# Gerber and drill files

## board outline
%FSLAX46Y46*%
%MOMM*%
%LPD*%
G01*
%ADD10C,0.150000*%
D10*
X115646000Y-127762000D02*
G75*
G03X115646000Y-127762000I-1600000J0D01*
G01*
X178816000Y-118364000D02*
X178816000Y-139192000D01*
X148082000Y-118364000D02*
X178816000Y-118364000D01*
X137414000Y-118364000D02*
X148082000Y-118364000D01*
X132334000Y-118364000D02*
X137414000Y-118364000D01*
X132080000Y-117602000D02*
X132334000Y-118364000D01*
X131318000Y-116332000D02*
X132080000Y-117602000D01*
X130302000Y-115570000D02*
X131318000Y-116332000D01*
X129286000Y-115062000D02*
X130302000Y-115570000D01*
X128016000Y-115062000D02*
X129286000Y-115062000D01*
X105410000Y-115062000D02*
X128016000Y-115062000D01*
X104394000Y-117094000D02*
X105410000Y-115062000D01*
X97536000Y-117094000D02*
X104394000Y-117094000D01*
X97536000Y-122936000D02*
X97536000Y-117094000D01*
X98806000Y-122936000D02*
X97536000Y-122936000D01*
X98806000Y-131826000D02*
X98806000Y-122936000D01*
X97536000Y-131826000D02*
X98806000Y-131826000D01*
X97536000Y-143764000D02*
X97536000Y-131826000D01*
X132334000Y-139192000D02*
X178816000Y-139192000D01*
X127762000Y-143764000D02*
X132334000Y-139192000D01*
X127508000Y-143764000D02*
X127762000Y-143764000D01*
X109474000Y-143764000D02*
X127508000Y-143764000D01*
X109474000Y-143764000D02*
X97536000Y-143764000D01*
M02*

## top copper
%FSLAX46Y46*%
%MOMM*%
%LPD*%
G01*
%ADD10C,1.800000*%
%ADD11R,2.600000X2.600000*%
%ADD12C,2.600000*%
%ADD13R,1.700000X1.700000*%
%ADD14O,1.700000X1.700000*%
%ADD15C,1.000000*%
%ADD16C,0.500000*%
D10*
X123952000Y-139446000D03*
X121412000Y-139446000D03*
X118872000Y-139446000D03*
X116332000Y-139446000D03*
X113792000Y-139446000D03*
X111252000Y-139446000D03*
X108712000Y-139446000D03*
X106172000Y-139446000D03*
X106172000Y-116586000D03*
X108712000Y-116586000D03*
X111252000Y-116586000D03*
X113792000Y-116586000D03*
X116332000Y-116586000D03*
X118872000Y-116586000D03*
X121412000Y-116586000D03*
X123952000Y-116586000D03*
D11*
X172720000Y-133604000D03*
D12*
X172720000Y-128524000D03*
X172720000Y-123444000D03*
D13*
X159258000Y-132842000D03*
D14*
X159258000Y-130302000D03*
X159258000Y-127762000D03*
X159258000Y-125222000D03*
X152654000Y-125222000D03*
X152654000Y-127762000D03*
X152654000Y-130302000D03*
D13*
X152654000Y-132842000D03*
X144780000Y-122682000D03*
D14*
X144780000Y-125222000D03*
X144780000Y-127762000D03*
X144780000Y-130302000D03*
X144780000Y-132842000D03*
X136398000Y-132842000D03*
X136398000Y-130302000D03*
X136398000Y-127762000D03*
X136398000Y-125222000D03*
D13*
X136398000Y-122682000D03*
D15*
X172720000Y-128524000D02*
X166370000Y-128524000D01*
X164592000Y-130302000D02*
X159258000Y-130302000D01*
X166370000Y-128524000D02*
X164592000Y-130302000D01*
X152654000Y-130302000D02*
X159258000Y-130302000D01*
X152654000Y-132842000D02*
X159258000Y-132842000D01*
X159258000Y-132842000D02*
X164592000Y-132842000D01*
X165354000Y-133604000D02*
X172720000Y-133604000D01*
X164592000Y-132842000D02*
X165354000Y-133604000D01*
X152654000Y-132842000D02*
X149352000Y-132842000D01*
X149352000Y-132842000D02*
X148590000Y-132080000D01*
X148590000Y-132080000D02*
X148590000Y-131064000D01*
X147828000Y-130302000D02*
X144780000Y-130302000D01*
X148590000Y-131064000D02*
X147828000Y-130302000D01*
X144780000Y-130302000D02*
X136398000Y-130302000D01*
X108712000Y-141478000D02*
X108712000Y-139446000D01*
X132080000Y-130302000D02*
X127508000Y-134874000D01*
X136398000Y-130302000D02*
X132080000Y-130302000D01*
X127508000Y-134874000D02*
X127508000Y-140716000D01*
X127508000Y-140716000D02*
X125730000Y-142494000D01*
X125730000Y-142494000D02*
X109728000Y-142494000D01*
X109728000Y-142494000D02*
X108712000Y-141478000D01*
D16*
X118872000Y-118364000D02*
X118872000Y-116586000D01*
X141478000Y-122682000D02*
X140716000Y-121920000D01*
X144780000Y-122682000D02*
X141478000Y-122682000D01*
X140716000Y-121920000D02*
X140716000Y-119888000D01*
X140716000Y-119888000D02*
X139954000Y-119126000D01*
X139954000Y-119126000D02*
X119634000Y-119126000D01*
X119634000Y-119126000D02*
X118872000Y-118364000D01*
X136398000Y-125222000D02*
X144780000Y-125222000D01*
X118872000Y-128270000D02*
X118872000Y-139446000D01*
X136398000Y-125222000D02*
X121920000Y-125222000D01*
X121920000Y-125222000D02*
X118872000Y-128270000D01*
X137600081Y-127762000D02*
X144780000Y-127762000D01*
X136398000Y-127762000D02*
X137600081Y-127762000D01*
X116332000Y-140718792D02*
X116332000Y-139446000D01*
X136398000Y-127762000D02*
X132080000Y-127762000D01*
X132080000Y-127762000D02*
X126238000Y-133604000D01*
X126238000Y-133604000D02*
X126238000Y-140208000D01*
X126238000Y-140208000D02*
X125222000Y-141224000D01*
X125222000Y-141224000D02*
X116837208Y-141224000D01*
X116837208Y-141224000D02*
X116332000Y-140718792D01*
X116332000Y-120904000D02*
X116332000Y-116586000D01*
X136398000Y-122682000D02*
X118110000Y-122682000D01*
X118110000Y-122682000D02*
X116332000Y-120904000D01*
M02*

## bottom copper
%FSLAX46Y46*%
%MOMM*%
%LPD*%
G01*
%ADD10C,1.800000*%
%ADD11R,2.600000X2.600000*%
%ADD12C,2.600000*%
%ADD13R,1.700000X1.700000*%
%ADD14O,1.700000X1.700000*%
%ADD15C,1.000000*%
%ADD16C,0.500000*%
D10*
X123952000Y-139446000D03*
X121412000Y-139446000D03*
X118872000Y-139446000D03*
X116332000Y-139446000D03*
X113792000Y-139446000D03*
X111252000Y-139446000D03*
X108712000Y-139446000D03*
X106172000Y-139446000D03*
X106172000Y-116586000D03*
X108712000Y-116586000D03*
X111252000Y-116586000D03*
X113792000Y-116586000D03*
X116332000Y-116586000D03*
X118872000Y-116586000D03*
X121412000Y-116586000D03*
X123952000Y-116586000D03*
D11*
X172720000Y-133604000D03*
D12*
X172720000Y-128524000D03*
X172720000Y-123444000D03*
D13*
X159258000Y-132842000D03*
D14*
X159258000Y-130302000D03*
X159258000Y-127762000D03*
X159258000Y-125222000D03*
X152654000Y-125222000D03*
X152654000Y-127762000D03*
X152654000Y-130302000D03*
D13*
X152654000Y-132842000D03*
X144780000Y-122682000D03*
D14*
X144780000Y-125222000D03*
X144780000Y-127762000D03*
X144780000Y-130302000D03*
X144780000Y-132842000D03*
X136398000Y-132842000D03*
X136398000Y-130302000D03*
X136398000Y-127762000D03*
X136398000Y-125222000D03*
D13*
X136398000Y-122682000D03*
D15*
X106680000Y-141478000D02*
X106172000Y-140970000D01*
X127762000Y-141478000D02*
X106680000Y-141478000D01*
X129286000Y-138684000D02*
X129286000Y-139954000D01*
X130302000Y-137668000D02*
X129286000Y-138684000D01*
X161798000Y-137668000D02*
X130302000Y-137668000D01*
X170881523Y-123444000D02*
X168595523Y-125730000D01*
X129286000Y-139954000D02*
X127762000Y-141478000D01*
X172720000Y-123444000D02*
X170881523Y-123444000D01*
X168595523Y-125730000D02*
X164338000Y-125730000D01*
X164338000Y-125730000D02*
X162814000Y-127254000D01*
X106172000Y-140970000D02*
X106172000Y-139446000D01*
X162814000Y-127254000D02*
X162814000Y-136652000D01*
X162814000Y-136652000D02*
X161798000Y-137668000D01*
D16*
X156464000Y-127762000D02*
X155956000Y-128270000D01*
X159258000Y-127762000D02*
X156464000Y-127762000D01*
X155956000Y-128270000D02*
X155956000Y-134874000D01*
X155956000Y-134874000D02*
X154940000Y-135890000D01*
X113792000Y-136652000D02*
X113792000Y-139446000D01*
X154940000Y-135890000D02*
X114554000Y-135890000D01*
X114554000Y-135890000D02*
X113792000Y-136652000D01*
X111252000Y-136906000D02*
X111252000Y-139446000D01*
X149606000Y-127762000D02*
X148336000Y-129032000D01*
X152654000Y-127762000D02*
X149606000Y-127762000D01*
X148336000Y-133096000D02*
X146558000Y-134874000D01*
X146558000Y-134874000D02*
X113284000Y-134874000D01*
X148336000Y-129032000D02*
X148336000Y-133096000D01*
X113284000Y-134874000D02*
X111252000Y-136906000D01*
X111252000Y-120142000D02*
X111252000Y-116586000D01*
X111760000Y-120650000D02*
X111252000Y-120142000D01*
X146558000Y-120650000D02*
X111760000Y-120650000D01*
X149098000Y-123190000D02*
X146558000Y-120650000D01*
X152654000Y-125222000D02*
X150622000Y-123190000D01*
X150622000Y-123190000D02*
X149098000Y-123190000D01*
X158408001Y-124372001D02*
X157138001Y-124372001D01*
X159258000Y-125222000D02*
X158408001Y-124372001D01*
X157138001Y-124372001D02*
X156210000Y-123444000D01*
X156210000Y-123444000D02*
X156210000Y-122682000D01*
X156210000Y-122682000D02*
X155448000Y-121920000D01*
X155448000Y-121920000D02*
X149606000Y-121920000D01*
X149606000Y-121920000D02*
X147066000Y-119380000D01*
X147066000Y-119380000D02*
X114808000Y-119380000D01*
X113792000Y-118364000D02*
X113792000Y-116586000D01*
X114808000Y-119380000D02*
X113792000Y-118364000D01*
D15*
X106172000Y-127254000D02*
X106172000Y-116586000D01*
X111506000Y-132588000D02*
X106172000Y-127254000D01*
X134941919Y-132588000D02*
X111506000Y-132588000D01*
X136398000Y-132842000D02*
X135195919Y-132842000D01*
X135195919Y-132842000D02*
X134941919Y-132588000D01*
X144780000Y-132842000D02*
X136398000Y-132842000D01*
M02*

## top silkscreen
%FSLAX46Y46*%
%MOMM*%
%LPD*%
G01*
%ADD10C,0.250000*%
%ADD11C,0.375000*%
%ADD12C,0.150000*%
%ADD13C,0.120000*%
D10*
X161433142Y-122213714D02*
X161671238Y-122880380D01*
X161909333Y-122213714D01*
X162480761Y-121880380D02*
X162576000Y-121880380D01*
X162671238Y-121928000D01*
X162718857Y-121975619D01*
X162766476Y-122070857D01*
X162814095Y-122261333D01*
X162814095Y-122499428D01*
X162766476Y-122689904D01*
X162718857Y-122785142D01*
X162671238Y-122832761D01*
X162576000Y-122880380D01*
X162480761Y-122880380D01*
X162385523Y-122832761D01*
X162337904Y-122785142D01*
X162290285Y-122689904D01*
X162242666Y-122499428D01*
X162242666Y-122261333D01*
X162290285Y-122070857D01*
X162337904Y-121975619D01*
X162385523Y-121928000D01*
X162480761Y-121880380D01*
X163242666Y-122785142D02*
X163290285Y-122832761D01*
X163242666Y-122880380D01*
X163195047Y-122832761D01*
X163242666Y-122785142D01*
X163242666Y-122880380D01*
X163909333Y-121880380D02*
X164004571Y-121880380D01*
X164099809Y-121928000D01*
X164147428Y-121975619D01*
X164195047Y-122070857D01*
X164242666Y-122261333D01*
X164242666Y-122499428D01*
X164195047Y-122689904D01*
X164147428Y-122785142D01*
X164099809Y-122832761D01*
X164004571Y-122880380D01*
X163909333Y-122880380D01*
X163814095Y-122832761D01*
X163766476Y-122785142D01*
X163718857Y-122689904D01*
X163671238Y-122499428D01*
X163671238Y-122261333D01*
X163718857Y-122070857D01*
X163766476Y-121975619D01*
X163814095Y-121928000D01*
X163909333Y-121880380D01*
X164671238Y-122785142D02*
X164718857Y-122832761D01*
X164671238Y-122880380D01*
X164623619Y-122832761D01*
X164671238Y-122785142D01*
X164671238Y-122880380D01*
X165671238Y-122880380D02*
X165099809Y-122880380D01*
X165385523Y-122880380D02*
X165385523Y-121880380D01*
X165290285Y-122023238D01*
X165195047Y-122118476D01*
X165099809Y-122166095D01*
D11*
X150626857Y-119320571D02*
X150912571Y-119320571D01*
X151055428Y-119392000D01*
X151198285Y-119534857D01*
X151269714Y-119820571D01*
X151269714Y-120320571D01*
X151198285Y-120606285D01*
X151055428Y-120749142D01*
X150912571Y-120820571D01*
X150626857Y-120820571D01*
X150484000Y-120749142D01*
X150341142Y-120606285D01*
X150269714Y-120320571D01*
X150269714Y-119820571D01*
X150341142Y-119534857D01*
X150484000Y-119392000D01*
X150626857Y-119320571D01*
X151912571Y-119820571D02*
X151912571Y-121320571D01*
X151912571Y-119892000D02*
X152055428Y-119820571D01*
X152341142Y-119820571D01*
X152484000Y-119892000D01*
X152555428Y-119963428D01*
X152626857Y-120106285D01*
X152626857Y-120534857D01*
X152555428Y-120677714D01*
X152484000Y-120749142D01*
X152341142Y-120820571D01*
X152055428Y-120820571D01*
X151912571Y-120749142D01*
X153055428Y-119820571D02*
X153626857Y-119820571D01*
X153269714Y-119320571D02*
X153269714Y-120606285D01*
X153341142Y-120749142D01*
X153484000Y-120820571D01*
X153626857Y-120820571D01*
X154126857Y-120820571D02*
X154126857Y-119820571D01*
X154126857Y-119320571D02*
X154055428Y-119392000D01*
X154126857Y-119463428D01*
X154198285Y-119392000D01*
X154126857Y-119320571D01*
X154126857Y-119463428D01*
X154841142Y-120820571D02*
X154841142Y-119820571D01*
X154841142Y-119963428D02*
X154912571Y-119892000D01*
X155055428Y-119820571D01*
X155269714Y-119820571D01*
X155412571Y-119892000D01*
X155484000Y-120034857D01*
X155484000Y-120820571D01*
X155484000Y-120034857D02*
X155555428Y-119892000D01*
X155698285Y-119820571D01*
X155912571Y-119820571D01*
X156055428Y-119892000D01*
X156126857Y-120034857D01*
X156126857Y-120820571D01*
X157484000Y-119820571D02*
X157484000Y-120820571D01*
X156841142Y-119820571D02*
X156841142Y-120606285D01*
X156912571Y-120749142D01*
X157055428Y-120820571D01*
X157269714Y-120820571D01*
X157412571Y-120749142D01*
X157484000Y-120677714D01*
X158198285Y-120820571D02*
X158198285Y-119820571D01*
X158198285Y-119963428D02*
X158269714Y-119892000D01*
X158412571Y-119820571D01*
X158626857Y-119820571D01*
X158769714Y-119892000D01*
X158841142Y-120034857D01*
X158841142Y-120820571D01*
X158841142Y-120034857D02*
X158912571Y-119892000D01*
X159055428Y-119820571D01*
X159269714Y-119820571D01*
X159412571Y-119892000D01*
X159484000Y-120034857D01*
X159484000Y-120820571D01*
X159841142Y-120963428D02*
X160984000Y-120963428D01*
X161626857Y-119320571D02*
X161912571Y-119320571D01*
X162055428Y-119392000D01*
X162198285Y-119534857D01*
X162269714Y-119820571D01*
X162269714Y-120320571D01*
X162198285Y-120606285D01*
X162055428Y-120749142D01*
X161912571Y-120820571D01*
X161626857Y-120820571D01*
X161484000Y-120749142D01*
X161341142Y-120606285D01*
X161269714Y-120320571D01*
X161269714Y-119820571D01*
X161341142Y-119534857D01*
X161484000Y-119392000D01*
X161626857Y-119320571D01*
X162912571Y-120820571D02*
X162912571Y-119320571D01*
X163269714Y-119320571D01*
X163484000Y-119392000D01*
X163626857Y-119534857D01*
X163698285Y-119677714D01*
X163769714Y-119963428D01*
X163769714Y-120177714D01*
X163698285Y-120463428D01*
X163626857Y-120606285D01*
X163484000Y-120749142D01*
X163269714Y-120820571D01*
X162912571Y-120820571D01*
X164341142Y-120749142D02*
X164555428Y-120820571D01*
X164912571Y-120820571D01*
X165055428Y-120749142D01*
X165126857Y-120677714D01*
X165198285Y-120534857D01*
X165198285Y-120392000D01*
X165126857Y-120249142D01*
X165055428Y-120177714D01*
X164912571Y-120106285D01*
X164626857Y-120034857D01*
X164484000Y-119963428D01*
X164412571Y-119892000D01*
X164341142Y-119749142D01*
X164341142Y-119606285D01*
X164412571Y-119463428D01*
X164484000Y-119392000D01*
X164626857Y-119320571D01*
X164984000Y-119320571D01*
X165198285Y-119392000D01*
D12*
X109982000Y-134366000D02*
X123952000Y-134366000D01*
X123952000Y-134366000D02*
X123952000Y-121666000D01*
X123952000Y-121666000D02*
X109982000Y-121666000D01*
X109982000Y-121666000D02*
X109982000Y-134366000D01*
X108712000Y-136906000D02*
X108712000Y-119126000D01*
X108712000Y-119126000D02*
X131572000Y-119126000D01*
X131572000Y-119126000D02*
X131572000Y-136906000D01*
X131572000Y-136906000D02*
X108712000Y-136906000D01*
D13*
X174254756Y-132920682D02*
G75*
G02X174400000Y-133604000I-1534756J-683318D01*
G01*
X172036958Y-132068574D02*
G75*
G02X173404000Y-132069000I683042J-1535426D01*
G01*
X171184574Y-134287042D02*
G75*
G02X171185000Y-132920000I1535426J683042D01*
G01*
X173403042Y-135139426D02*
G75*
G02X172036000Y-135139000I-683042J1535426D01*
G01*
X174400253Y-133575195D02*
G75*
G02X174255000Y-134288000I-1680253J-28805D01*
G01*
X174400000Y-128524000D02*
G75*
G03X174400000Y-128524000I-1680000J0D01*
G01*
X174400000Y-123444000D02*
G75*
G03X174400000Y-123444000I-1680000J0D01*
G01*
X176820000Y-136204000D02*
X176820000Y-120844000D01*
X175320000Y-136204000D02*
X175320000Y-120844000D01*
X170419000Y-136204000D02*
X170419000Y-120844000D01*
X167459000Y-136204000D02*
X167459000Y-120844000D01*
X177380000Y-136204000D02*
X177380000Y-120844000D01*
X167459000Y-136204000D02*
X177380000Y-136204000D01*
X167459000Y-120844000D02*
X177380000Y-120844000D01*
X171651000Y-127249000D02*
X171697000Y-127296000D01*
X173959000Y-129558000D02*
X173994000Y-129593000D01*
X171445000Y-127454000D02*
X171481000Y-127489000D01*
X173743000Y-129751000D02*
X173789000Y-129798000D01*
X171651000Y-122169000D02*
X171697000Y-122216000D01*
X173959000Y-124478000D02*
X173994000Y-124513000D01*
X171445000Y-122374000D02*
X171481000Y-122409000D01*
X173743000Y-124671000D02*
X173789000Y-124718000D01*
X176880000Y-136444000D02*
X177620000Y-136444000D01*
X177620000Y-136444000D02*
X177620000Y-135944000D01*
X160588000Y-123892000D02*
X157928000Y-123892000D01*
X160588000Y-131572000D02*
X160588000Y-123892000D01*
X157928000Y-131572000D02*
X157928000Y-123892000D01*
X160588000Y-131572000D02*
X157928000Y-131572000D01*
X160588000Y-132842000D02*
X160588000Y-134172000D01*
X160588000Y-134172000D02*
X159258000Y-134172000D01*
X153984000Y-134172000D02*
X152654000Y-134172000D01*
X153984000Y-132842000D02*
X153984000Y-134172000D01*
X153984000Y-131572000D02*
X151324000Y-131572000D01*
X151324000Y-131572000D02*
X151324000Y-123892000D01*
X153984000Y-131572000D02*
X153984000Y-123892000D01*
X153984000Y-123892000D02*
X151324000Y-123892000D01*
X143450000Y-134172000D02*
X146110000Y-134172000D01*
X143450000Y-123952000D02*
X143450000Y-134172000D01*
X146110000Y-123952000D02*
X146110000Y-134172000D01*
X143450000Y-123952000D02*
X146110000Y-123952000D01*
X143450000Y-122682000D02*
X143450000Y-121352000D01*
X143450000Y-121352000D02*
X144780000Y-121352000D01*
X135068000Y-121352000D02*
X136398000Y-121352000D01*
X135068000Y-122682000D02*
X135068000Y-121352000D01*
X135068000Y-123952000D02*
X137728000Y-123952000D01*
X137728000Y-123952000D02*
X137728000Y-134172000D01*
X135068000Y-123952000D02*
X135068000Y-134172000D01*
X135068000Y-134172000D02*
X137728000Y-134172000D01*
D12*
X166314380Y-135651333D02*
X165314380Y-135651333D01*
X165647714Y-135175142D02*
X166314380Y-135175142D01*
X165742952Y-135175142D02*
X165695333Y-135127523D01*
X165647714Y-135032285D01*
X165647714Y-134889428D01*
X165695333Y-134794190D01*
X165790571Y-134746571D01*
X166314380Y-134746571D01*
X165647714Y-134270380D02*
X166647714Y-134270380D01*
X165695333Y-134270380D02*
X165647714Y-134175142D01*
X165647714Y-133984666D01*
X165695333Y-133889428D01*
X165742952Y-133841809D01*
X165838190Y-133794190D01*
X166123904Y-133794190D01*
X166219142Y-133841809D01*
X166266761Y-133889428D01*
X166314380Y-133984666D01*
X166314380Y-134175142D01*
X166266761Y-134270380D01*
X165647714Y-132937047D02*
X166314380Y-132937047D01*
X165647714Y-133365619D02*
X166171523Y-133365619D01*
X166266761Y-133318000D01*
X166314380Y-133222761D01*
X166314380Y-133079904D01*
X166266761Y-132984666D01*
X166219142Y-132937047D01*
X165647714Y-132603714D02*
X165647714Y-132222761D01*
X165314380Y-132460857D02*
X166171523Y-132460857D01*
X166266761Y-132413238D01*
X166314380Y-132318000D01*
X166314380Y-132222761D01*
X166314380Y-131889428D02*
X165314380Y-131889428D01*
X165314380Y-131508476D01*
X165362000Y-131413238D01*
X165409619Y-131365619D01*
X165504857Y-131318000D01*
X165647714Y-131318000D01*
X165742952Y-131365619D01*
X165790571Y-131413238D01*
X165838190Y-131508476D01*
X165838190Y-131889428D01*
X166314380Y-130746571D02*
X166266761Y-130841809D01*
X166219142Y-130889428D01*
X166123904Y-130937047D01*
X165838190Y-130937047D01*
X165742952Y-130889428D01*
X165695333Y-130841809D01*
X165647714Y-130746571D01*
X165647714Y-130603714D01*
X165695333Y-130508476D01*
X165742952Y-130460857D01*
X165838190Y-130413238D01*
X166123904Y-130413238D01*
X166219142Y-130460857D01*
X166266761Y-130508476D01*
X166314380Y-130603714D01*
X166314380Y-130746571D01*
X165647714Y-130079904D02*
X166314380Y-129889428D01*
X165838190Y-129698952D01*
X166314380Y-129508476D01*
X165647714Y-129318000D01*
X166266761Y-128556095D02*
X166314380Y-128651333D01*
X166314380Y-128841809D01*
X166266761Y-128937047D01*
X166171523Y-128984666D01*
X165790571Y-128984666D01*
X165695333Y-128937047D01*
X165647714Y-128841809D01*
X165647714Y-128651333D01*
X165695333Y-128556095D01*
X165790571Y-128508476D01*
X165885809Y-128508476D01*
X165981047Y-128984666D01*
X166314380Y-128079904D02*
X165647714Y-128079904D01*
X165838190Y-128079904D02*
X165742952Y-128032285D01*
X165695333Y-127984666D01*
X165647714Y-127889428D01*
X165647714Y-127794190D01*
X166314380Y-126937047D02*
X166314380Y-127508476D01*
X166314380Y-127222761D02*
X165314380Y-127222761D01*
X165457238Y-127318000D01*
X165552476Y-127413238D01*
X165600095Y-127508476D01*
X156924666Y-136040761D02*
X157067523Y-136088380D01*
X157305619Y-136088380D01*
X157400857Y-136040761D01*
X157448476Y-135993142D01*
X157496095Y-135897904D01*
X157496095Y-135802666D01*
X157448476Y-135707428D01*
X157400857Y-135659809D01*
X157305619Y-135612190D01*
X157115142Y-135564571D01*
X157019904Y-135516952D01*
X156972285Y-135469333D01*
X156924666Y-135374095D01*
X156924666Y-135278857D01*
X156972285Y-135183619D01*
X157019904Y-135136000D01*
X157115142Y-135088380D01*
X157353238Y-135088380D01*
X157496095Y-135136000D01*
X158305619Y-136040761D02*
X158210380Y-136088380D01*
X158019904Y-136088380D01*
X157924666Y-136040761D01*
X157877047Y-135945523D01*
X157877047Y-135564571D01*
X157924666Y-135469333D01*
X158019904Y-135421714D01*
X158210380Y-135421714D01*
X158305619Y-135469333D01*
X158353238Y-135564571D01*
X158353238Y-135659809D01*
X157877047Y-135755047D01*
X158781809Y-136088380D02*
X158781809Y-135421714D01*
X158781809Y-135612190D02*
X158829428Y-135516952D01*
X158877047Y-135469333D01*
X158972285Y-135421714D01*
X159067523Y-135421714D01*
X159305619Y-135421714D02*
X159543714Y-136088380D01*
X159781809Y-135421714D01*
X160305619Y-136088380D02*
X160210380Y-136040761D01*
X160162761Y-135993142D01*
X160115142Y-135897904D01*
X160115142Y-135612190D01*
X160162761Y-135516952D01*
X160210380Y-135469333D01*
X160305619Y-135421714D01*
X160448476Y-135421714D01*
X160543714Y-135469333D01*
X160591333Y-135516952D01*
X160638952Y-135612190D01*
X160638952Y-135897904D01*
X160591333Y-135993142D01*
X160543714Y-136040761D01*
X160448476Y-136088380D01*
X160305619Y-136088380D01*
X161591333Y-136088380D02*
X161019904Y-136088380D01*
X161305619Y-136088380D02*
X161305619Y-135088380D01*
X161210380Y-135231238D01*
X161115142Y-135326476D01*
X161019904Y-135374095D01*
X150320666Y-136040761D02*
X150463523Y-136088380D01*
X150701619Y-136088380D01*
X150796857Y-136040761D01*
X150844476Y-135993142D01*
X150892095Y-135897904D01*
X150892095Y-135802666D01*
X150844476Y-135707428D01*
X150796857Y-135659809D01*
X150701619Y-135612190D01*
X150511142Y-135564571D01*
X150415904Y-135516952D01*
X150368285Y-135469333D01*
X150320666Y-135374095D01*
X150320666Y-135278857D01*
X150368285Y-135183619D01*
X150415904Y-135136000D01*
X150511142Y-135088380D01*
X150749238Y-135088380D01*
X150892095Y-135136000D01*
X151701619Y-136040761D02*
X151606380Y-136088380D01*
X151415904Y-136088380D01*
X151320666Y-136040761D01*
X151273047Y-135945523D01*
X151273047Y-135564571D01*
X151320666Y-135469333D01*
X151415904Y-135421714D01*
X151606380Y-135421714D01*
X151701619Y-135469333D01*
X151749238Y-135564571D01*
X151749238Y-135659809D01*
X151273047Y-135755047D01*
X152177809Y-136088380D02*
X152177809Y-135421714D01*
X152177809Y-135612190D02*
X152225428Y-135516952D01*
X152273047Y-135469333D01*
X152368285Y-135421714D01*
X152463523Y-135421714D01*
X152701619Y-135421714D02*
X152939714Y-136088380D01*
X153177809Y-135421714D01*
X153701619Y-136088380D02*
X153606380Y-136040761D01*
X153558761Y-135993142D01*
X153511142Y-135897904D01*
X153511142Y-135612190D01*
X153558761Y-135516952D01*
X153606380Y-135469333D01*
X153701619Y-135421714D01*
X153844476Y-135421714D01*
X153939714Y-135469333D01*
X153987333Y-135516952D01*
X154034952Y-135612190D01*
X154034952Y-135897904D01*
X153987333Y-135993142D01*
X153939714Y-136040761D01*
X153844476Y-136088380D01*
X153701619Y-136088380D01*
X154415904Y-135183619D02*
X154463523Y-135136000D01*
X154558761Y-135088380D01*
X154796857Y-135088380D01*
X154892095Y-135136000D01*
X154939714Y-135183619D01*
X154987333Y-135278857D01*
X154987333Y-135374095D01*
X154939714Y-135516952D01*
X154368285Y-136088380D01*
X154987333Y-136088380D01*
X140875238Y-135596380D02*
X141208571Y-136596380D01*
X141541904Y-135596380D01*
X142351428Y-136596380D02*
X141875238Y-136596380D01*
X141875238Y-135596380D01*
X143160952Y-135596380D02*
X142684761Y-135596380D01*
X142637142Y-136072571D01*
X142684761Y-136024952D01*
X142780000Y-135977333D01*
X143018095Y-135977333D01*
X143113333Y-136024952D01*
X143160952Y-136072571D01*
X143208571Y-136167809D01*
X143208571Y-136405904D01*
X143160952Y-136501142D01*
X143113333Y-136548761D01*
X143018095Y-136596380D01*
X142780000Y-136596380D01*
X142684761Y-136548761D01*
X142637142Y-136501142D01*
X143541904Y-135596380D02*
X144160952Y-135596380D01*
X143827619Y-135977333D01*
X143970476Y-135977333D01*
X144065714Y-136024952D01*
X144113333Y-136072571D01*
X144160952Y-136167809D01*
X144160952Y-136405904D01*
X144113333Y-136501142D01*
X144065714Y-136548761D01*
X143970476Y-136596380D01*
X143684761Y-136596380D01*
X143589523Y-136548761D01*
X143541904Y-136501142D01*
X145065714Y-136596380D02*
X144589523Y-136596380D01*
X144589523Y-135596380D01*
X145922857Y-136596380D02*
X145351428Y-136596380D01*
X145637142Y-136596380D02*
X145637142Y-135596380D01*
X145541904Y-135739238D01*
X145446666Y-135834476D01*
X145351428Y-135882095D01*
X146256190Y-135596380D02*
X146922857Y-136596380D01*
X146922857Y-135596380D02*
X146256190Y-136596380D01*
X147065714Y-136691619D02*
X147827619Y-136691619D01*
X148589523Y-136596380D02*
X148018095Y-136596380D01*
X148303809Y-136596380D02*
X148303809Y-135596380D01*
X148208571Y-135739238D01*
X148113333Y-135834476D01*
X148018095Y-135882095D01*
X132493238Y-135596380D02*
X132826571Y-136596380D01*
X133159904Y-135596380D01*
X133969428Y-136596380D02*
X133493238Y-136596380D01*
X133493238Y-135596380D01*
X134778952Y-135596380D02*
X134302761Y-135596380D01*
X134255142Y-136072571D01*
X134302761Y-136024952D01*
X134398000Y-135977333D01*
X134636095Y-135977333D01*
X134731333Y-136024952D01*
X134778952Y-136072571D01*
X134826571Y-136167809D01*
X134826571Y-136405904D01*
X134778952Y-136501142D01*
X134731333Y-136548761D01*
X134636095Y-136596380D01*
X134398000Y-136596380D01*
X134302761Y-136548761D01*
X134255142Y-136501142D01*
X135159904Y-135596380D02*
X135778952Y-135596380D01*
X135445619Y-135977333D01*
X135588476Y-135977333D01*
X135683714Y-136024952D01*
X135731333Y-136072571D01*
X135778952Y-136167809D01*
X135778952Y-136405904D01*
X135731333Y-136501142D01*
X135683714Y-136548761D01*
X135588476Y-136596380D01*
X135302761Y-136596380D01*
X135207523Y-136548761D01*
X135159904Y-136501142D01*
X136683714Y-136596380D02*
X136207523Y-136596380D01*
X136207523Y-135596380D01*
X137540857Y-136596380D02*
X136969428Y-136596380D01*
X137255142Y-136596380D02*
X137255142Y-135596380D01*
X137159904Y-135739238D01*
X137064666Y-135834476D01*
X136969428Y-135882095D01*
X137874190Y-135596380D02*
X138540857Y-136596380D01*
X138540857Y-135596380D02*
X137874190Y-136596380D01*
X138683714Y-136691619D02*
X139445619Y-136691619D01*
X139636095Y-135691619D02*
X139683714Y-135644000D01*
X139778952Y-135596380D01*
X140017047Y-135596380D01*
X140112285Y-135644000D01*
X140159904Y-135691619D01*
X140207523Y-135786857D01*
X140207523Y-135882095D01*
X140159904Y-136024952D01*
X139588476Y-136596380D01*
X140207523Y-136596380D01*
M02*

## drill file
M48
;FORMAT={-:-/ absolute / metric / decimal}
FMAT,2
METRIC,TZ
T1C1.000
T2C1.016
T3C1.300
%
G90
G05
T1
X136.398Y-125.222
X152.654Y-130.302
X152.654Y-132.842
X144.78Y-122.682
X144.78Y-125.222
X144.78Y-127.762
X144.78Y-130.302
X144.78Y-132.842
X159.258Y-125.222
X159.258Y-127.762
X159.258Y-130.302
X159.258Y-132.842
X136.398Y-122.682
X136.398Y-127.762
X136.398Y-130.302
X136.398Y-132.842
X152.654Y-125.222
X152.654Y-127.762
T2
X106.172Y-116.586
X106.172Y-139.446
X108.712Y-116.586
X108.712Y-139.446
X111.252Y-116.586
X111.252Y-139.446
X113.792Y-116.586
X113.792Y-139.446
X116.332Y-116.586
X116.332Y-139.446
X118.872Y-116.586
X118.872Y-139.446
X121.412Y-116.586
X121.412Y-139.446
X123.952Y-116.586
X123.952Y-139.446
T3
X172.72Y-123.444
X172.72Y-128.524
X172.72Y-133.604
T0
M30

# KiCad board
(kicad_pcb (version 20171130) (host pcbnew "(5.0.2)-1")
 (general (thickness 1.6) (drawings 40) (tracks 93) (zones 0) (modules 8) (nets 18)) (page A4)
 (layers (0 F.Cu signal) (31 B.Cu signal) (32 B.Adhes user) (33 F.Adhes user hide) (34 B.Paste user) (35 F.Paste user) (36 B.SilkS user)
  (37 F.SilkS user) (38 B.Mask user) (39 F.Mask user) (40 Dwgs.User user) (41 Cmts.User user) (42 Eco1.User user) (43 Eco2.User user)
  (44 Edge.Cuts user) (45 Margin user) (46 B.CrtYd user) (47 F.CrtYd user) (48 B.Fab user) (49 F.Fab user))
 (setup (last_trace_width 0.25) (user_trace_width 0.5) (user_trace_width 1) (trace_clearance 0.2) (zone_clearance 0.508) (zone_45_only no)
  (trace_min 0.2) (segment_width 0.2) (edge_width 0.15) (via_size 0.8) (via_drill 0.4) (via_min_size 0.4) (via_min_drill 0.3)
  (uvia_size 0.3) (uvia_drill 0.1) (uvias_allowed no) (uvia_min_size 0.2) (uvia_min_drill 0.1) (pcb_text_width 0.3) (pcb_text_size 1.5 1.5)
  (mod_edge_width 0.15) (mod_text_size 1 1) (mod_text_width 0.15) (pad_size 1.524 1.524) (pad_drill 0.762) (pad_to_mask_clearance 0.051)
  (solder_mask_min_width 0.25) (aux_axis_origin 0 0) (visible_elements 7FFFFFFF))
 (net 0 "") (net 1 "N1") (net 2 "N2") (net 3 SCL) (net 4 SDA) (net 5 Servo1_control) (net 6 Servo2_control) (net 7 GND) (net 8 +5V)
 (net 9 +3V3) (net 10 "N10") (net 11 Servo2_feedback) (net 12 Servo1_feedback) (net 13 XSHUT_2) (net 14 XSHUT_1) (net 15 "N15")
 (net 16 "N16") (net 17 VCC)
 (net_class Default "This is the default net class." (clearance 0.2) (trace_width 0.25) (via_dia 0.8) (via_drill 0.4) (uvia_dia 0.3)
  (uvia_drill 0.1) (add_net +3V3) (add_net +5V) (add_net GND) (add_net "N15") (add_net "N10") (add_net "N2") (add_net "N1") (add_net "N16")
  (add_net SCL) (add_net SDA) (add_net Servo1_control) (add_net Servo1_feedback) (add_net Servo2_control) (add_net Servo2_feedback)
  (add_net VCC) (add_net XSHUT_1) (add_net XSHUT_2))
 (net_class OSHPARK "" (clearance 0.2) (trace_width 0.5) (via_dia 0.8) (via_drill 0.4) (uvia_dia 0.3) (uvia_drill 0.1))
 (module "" (layer F.Cu) (at 156.464 121.666)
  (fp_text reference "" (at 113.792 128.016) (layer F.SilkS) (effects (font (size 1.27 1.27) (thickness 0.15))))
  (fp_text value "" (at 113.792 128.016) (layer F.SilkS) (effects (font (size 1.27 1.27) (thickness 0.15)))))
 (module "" (layer F.Cu) (at 156.972 120.142)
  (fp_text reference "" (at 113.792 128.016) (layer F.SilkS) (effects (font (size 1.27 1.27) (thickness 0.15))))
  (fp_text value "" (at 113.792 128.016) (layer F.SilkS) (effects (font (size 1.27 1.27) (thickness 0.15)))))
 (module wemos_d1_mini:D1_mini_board (layer B.Cu) (at 113.792 128.016 90)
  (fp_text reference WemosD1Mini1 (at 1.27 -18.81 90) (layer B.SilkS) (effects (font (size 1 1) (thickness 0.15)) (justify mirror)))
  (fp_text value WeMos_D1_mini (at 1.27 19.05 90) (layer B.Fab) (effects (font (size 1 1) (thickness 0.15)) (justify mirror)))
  (fp_line (start -6.35 -3.81) (end -6.35 10.16) (layer F.SilkS) (width 0.15))
  (fp_line (start -6.35 10.16) (end 6.35 10.16) (layer F.SilkS) (width 0.15))
  (fp_line (start 6.35 10.16) (end 6.35 -3.81) (layer F.SilkS) (width 0.15))
  (fp_line (start 6.35 -3.81) (end -6.35 -3.81) (layer F.SilkS) (width 0.15))
  (fp_line (start -8.89 -5.08) (end 8.89 -5.08) (layer F.SilkS) (width 0.15))
  (fp_line (start 8.89 -5.08) (end 8.89 17.78) (layer F.SilkS) (width 0.15))
  (fp_line (start 8.89 17.78) (end -8.89 17.78) (layer F.SilkS) (width 0.15))
  (fp_line (start -8.89 17.78) (end -8.89 -5.08) (layer F.SilkS) (width 0.15))
  (pad 8 thru_hole circle (at -11.43 10.16 90) (size 1.8 1.8) (drill 1.016) (layers *.Cu *.Mask B.SilkS) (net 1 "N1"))
  (pad 7 thru_hole circle (at -11.43 7.62 90) (size 1.8 1.8) (drill 1.016) (layers *.Cu *.Mask B.SilkS) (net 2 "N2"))
  (pad 6 thru_hole circle (at -11.43 5.08 90) (size 1.8 1.8) (drill 1.016) (layers *.Cu *.Mask B.SilkS) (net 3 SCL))
  (pad 5 thru_hole circle (at -11.43 2.54 90) (size 1.8 1.8) (drill 1.016) (layers *.Cu *.Mask B.SilkS) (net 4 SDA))
  (pad 4 thru_hole circle (at -11.43 0 90) (size 1.8 1.8) (drill 1.016) (layers *.Cu *.Mask B.SilkS) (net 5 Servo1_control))
  (pad 3 thru_hole circle (at -11.43 -2.54 90) (size 1.8 1.8) (drill 1.016) (layers *.Cu *.Mask B.SilkS) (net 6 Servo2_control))
  (pad 2 thru_hole circle (at -11.43 -5.08 90) (size 1.8 1.8) (drill 1.016) (layers *.Cu *.Mask B.SilkS) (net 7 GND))
  (pad 1 thru_hole circle (at -11.43 -7.62 90) (size 1.8 1.8) (drill 1.016) (layers *.Cu *.Mask B.SilkS) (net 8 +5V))
  (pad 16 thru_hole circle (at 11.43 -7.62 90) (size 1.8 1.8) (drill 1.016) (layers *.Cu *.Mask B.SilkS) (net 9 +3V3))
  (pad 15 thru_hole circle (at 11.43 -5.08 90) (size 1.8 1.8) (drill 1.016) (layers *.Cu *.Mask B.SilkS) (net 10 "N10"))
  (pad 14 thru_hole circle (at 11.43 -2.54 90) (size 1.8 1.8) (drill 1.016) (layers *.Cu *.Mask B.SilkS) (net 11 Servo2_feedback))
  (pad 13 thru_hole circle (at 11.43 0 90) (size 1.8 1.8) (drill 1.016) (layers *.Cu *.Mask B.SilkS) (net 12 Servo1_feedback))
  (pad 12 thru_hole circle (at 11.43 2.54 90) (size 1.8 1.8) (drill 1.016) (layers *.Cu *.Mask B.SilkS) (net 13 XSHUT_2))
  (pad 11 thru_hole circle (at 11.43 5.08 90) (size 1.8 1.8) (drill 1.016) (layers *.Cu *.Mask B.SilkS) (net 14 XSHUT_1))
  (pad 10 thru_hole circle (at 11.43 7.62 90) (size 1.8 1.8) (drill 1.016) (layers *.Cu *.Mask B.SilkS) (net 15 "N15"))
  (pad 9 thru_hole circle (at 11.43 10.16 90) (size 1.8 1.8) (drill 1.016) (layers *.Cu *.Mask B.SilkS) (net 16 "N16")))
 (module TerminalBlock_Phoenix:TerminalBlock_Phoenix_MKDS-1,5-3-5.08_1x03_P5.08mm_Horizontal (layer F.Cu) (at 172.72 133.604 90)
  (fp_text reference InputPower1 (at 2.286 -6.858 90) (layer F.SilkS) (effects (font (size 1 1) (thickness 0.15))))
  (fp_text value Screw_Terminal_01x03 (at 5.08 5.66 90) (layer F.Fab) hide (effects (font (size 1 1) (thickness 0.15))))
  (fp_arc (start 0 0) (end 0 1.68) (angle -24) (layer F.SilkS) (width 0.12))
  (fp_arc (start 0 0) (end 1.535 0.684) (angle -48) (layer F.SilkS) (width 0.12))
  (fp_arc (start 0 0) (end 0.684 -1.535) (angle -48) (layer F.SilkS) (width 0.12))
  (fp_arc (start 0 0) (end -1.535 -0.684) (angle -48) (layer F.SilkS) (width 0.12))
  (fp_arc (start 0 0) (end -0.684 1.535) (angle -25) (layer F.SilkS) (width 0.12))
  (fp_circle (center 5.08 0) (end 6.76 0) (layer F.SilkS) (width 0.12))
  (fp_circle (center 10.16 0) (end 11.84 0) (layer F.SilkS) (width 0.12))
  (fp_line (start -2.6 4.1) (end 12.76 4.1) (layer F.SilkS) (width 0.12))
  (fp_line (start -2.6 2.6) (end 12.76 2.6) (layer F.SilkS) (width 0.12))
  (fp_line (start -2.6 -2.301) (end 12.76 -2.301) (layer F.SilkS) (width 0.12))
  (fp_line (start -2.6 -5.261) (end 12.76 -5.261) (layer F.SilkS) (width 0.12))
  (fp_line (start -2.6 4.66) (end 12.76 4.66) (layer F.SilkS) (width 0.12))
  (fp_line (start -2.6 -5.261) (end -2.6 4.66) (layer F.SilkS) (width 0.12))
  (fp_line (start 12.76 -5.261) (end 12.76 4.66) (layer F.SilkS) (width 0.12))
  (fp_line (start 6.355 -1.069) (end 6.308 -1.023) (layer F.SilkS) (width 0.12))
  (fp_line (start 4.046 1.239) (end 4.011 1.274) (layer F.SilkS) (width 0.12))
  (fp_line (start 6.15 -1.275) (end 6.115 -1.239) (layer F.SilkS) (width 0.12))
  (fp_line (start 3.853 1.023) (end 3.806 1.069) (layer F.SilkS) (width 0.12))
  (fp_line (start 11.435 -1.069) (end 11.388 -1.023) (layer F.SilkS) (width 0.12))
  (fp_line (start 9.126 1.239) (end 9.091 1.274) (layer F.SilkS) (width 0.12))
  (fp_line (start 11.23 -1.275) (end 11.195 -1.239) (layer F.SilkS) (width 0.12))
  (fp_line (start 8.933 1.023) (end 8.886 1.069) (layer F.SilkS) (width 0.12))
  (fp_line (start -2.84 4.16) (end -2.84 4.9) (layer F.SilkS) (width 0.12))
  (fp_line (start -2.84 4.9) (end -2.34 4.9) (layer F.SilkS) (width 0.12))
  (pad 1 thru_hole rect (at 0 0 90) (size 2.6 2.6) (drill 1.3) (layers *.Cu *.Mask) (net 7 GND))
  (pad 2 thru_hole circle (at 5.08 0 90) (size 2.6 2.6) (drill 1.3) (layers *.Cu *.Mask) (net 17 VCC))
  (pad 3 thru_hole circle (at 10.16 0 90) (size 2.6 2.6) (drill 1.3) (layers *.Cu *.Mask) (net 8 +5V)))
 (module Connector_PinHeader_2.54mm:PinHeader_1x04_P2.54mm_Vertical (layer F.Cu) (at 159.258 132.842 180)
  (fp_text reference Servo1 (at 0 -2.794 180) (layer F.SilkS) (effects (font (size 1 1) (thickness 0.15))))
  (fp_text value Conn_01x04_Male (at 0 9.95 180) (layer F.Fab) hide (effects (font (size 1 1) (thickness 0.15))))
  (fp_line (start -1.33 8.95) (end 1.33 8.95) (layer F.SilkS) (width 0.12))
  (fp_line (start -1.33 1.27) (end -1.33 8.95) (layer F.SilkS) (width 0.12))
  (fp_line (start 1.33 1.27) (end 1.33 8.95) (layer F.SilkS) (width 0.12))
  (fp_line (start -1.33 1.27) (end 1.33 1.27) (layer F.SilkS) (width 0.12))
  (fp_line (start -1.33 0) (end -1.33 -1.33) (layer F.SilkS) (width 0.12))
  (fp_line (start -1.33 -1.33) (end 0 -1.33) (layer F.SilkS) (width 0.12))
  (pad 1 thru_hole rect (at 0 0 180) (size 1.7 1.7) (drill 1) (layers *.Cu *.Mask) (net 7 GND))
  (pad 2 thru_hole oval (at 0 2.54 180) (size 1.7 1.7) (drill 1) (layers *.Cu *.Mask) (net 17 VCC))
  (pad 3 thru_hole oval (at 0 5.08 180) (size 1.7 1.7) (drill 1) (layers *.Cu *.Mask) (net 5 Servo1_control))
  (pad 4 thru_hole oval (at 0 7.62 180) (size 1.7 1.7) (drill 1) (layers *.Cu *.Mask) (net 12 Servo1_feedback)))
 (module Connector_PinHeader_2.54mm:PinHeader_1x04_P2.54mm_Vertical (layer F.Cu) (at 152.654 132.842 180)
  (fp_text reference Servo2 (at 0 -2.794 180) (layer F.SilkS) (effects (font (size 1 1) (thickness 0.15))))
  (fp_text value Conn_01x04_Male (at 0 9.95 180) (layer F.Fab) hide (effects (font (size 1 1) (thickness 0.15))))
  (fp_line (start -1.33 -1.33) (end 0 -1.33) (layer F.SilkS) (width 0.12))
  (fp_line (start -1.33 0) (end -1.33 -1.33) (layer F.SilkS) (width 0.12))
  (fp_line (start -1.33 1.27) (end 1.33 1.27) (layer F.SilkS) (width 0.12))
  (fp_line (start 1.33 1.27) (end 1.33 8.95) (layer F.SilkS) (width 0.12))
  (fp_line (start -1.33 1.27) (end -1.33 8.95) (layer F.SilkS) (width 0.12))
  (fp_line (start -1.33 8.95) (end 1.33 8.95) (layer F.SilkS) (width 0.12))
  (pad 4 thru_hole oval (at 0 7.62 180) (size 1.7 1.7) (drill 1) (layers *.Cu *.Mask) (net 11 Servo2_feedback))
  (pad 3 thru_hole oval (at 0 5.08 180) (size 1.7 1.7) (drill 1) (layers *.Cu *.Mask) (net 6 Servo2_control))
  (pad 2 thru_hole oval (at 0 2.54 180) (size 1.7 1.7) (drill 1) (layers *.Cu *.Mask) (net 17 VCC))
  (pad 1 thru_hole rect (at 0 0 180) (size 1.7 1.7) (drill 1) (layers *.Cu *.Mask) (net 7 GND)))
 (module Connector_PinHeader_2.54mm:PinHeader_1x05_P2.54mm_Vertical (layer F.Cu) (at 144.78 122.682)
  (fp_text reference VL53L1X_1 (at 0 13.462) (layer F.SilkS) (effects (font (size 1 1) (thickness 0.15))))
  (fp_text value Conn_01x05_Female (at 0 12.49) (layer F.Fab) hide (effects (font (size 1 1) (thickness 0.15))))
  (fp_line (start -1.33 11.49) (end 1.33 11.49) (layer F.SilkS) (width 0.12))
  (fp_line (start -1.33 1.27) (end -1.33 11.49) (layer F.SilkS) (width 0.12))
  (fp_line (start 1.33 1.27) (end 1.33 11.49) (layer F.SilkS) (width 0.12))
  (fp_line (start -1.33 1.27) (end 1.33 1.27) (layer F.SilkS) (width 0.12))
  (fp_line (start -1.33 0) (end -1.33 -1.33) (layer F.SilkS) (width 0.12))
  (fp_line (start -1.33 -1.33) (end 0 -1.33) (layer F.SilkS) (width 0.12))
  (pad 1 thru_hole rect (at 0 0) (size 1.7 1.7) (drill 1) (layers *.Cu *.Mask) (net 14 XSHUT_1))
  (pad 2 thru_hole oval (at 0 2.54) (size 1.7 1.7) (drill 1) (layers *.Cu *.Mask) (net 3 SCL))
  (pad 3 thru_hole oval (at 0 5.08) (size 1.7 1.7) (drill 1) (layers *.Cu *.Mask) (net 4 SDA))
  (pad 4 thru_hole oval (at 0 7.62) (size 1.7 1.7) (drill 1) (layers *.Cu *.Mask) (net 7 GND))
  (pad 5 thru_hole oval (at 0 10.16) (size 1.7 1.7) (drill 1) (layers *.Cu *.Mask) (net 9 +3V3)))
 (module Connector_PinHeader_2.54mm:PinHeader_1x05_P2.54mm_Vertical (layer F.Cu) (at 136.398 122.682)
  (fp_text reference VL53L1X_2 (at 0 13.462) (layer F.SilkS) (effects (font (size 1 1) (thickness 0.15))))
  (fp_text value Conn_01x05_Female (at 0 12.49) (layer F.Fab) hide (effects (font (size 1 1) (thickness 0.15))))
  (fp_line (start -1.33 -1.33) (end 0 -1.33) (layer F.SilkS) (width 0.12))
  (fp_line (start -1.33 0) (end -1.33 -1.33) (layer F.SilkS) (width 0.12))
  (fp_line (start -1.33 1.27) (end 1.33 1.27) (layer F.SilkS) (width 0.12))
  (fp_line (start 1.33 1.27) (end 1.33 11.49) (layer F.SilkS) (width 0.12))
  (fp_line (start -1.33 1.27) (end -1.33 11.49) (layer F.SilkS) (width 0.12))
  (fp_line (start -1.33 11.49) (end 1.33 11.49) (layer F.SilkS) (width 0.12))
  (pad 5 thru_hole oval (at 0 10.16) (size 1.7 1.7) (drill 1) (layers *.Cu *.Mask) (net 9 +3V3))
  (pad 4 thru_hole oval (at 0 7.62) (size 1.7 1.7) (drill 1) (layers *.Cu *.Mask) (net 7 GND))
  (pad 3 thru_hole oval (at 0 5.08) (size 1.7 1.7) (drill 1) (layers *.Cu *.Mask) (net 4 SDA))
  (pad 2 thru_hole oval (at 0 2.54) (size 1.7 1.7) (drill 1) (layers *.Cu *.Mask) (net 3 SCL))
  (pad 1 thru_hole rect (at 0 0) (size 1.7 1.7) (drill 1) (layers *.Cu *.Mask) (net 13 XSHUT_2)))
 (gr_circle (center 114.046 127.762) (end 115.646 127.762) (layer Edge.Cuts) (width 0.15))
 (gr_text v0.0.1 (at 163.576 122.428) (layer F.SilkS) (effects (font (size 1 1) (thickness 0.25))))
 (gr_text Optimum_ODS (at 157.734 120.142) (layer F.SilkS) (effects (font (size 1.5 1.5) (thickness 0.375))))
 (gr_line (start 178.816 118.364) (end 178.816 139.192) (layer Edge.Cuts) (width 0.15))
 (gr_line (start 148.082 118.364) (end 178.816 118.364) (layer Edge.Cuts) (width 0.15))
 (gr_line (start 137.414 118.364) (end 148.082 118.364) (layer Edge.Cuts) (width 0.15))
 (gr_line (start 132.334 118.364) (end 137.414 118.364) (layer Edge.Cuts) (width 0.15))
 (gr_line (start 132.08 117.602) (end 132.334 118.364) (layer Edge.Cuts) (width 0.15))
 (gr_line (start 131.318 116.332) (end 132.08 117.602) (layer Edge.Cuts) (width 0.15))
 (gr_line (start 130.302 115.57) (end 131.318 116.332) (layer Edge.Cuts) (width 0.15))
 (gr_line (start 129.286 115.062) (end 130.302 115.57) (layer Edge.Cuts) (width 0.15))
 (gr_line (start 128.016 115.062) (end 129.286 115.062) (layer Edge.Cuts) (width 0.15))
 (gr_line (start 105.41 115.062) (end 128.016 115.062) (layer Edge.Cuts) (width 0.15))
 (gr_line (start 104.394 117.094) (end 105.41 115.062) (layer Edge.Cuts) (width 0.15))
 (gr_line (start 97.536 117.094) (end 104.394 117.094) (layer Edge.Cuts) (width 0.15))
 (gr_line (start 97.536 122.936) (end 97.536 117.094) (layer Edge.Cuts) (width 0.15))
 (gr_line (start 98.806 122.936) (end 97.536 122.936) (layer Edge.Cuts) (width 0.15))
 (gr_line (start 98.806 131.826) (end 98.806 122.936) (layer Edge.Cuts) (width 0.15))
 (gr_line (start 97.536 131.826) (end 98.806 131.826) (layer Edge.Cuts) (width 0.15))
 (gr_line (start 97.536 143.764) (end 97.536 131.826) (layer Edge.Cuts) (width 0.15))
 (gr_line (start 132.334 139.192) (end 178.816 139.192) (layer Edge.Cuts) (width 0.15))
 (gr_line (start 127.762 143.764) (end 132.334 139.192) (layer Edge.Cuts) (width 0.15))
 (gr_line (start 127.508 143.764) (end 127.762 143.764) (layer Edge.Cuts) (width 0.15))
 (gr_line (start 109.474 143.764) (end 127.508 143.764) (layer Edge.Cuts) (width 0.15))
 (gr_line (start 109.474 143.764) (end 97.536 143.764) (layer Edge.Cuts) (width 0.15))
 (segment (start 106.68 141.478) (end 106.172 140.97) (width 1) (layer B.Cu) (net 8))
 (segment (start 127.762 141.478) (end 106.68 141.478) (width 1) (layer B.Cu) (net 8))
 (segment (start 129.286 138.684) (end 129.286 139.954) (width 1) (layer B.Cu) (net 8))
 (segment (start 130.302 137.668) (end 129.286 138.684) (width 1) (layer B.Cu) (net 8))
 (segment (start 161.798 137.668) (end 130.302 137.668) (width 1) (layer B.Cu) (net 8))
 (segment (start 170.881523 123.444) (end 168.595523 125.73) (width 1) (layer B.Cu) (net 8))
 (segment (start 129.286 139.954) (end 127.762 141.478) (width 1) (layer B.Cu) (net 8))
 (segment (start 172.72 123.444) (end 170.881523 123.444) (width 1) (layer B.Cu) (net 8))
 (segment (start 168.595523 125.73) (end 164.338 125.73) (width 1) (layer B.Cu) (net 8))
 (segment (start 164.338 125.73) (end 162.814 127.254) (width 1) (layer B.Cu) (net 8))
 (segment (start 106.172 140.97) (end 106.172 139.446) (width 1) (layer B.Cu) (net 8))
 (segment (start 162.814 127.254) (end 162.814 136.652) (width 1) (layer B.Cu) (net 8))
 (segment (start 162.814 136.652) (end 161.798 137.668) (width 1) (layer B.Cu) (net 8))
 (segment (start 172.72 128.524) (end 166.37 128.524) (width 1) (layer F.Cu) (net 17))
 (segment (start 164.592 130.302) (end 159.258 130.302) (width 1) (layer F.Cu) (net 17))
 (segment (start 166.37 128.524) (end 164.592 130.302) (width 1) (layer F.Cu) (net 17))
 (segment (start 152.654 130.302) (end 159.258 130.302) (width 1) (layer F.Cu) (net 17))
 (segment (start 152.654 132.842) (end 159.258 132.842) (width 1) (layer F.Cu) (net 7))
 (segment (start 159.258 132.842) (end 164.592 132.842) (width 1) (layer F.Cu) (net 7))
 (segment (start 165.354 133.604) (end 172.72 133.604) (width 1) (layer F.Cu) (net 7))
 (segment (start 164.592 132.842) (end 165.354 133.604) (width 1) (layer F.Cu) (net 7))
 (segment (start 152.654 132.842) (end 149.352 132.842) (width 1) (layer F.Cu) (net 7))
 (segment (start 149.352 132.842) (end 148.59 132.08) (width 1) (layer F.Cu) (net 7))
 (segment (start 148.59 132.08) (end 148.59 131.064) (width 1) (layer F.Cu) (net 7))
 (segment (start 147.828 130.302) (end 144.78 130.302) (width 1) (layer F.Cu) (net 7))
 (segment (start 148.59 131.064) (end 147.828 130.302) (width 1) (layer F.Cu) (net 7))
 (segment (start 144.78 130.302) (end 136.398 130.302) (width 1) (layer F.Cu) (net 7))
 (segment (start 108.712 141.478) (end 108.712 139.446) (width 1) (layer F.Cu) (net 7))
 (segment (start 132.08 130.302) (end 127.508 134.874) (width 1) (layer F.Cu) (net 7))
 (segment (start 136.398 130.302) (end 132.08 130.302) (width 1) (layer F.Cu) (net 7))
 (segment (start 127.508 134.874) (end 127.508 140.716) (width 1) (layer F.Cu) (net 7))
 (segment (start 127.508 140.716) (end 125.73 142.494) (width 1) (layer F.Cu) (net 7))
 (segment (start 125.73 142.494) (end 109.728 142.494) (width 1) (layer F.Cu) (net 7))
 (segment (start 109.728 142.494) (end 108.712 141.478) (width 1) (layer F.Cu) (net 7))
 (segment (start 156.464 127.762) (end 155.956 128.27) (width 0.5) (layer B.Cu) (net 5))
 (segment (start 159.258 127.762) (end 156.464 127.762) (width 0.5) (layer B.Cu) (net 5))
 (segment (start 155.956 128.27) (end 155.956 134.874) (width 0.5) (layer B.Cu) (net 5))
 (segment (start 155.956 134.874) (end 154.94 135.89) (width 0.5) (layer B.Cu) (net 5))
 (segment (start 113.792 136.652) (end 113.792 139.446) (width 0.5) (layer B.Cu) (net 5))
 (segment (start 154.94 135.89) (end 114.554 135.89) (width 0.5) (layer B.Cu) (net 5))
 (segment (start 114.554 135.89) (end 113.792 136.652) (width 0.5) (layer B.Cu) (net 5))
 (segment (start 111.252 136.906) (end 111.252 139.446) (width 0.5) (layer B.Cu) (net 6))
 (segment (start 149.606 127.762) (end 148.336 129.032) (width 0.5) (layer B.Cu) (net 6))
 (segment (start 152.654 127.762) (end 149.606 127.762) (width 0.5) (layer B.Cu) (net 6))
 (segment (start 148.336 133.096) (end 146.558 134.874) (width 0.5) (layer B.Cu) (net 6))
 (segment (start 146.558 134.874) (end 113.284 134.874) (width 0.5) (layer B.Cu) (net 6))
 (segment (start 148.336 129.032) (end 148.336 133.096) (width 0.5) (layer B.Cu) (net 6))
 (segment (start 113.284 134.874) (end 111.252 136.906) (width 0.5) (layer B.Cu) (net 6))
 (segment (start 118.872 118.364) (end 118.872 116.586) (width 0.5) (layer F.Cu) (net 14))
 (segment (start 141.478 122.682) (end 140.716 121.92) (width 0.5) (layer F.Cu) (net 14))
 (segment (start 144.78 122.682) (end 141.478 122.682) (width 0.5) (layer F.Cu) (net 14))
 (segment (start 140.716 121.92) (end 140.716 119.888) (width 0.5) (layer F.Cu) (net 14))
 (segment (start 140.716 119.888) (end 139.954 119.126) (width 0.5) (layer F.Cu) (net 14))
 (segment (start 139.954 119.126) (end 119.634 119.126) (width 0.5) (layer F.Cu) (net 14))
 (segment (start 119.634 119.126) (end 118.872 118.364) (width 0.5) (layer F.Cu) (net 14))
 (segment (start 136.398 125.222) (end 144.78 125.222) (width 0.5) (layer F.Cu) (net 3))
 (segment (start 118.872 128.27) (end 118.872 139.446) (width 0.5) (layer F.Cu) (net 3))
 (segment (start 136.398 125.222) (end 121.92 125.222) (width 0.5) (layer F.Cu) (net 3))
 (segment (start 121.92 125.222) (end 118.872 128.27) (width 0.5) (layer F.Cu) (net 3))
 (segment (start 137.600081 127.762) (end 144.78 127.762) (width 0.5) (layer F.Cu) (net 4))
 (segment (start 136.398 127.762) (end 137.600081 127.762) (width 0.5) (layer F.Cu) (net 4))
 (segment (start 116.332 140.718792) (end 116.332 139.446) (width 0.5) (layer F.Cu) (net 4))
 (segment (start 136.398 127.762) (end 132.08 127.762) (width 0.5) (layer F.Cu) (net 4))
 (segment (start 132.08 127.762) (end 126.238 133.604) (width 0.5) (layer F.Cu) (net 4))
 (segment (start 126.238 133.604) (end 126.238 140.208) (width 0.5) (layer F.Cu) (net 4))
 (segment (start 126.238 140.208) (end 125.222 141.224) (width 0.5) (layer F.Cu) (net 4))
 (segment (start 125.222 141.224) (end 116.837208 141.224) (width 0.5) (layer F.Cu) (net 4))
 (segment (start 116.837208 141.224) (end 116.332 140.718792) (width 0.5) (layer F.Cu) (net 4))
 (segment (start 116.332 120.904) (end 116.332 116.586) (width 0.5) (layer F.Cu) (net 13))
 (segment (start 136.398 122.682) (end 118.11 122.682) (width 0.5) (layer F.Cu) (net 13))
 (segment (start 118.11 122.682) (end 116.332 120.904) (width 0.5) (layer F.Cu) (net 13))
 (segment (start 111.252 120.142) (end 111.252 116.586) (width 0.5) (layer B.Cu) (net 11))
 (segment (start 111.76 120.65) (end 111.252 120.142) (width 0.5) (layer B.Cu) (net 11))
 (segment (start 146.558 120.65) (end 111.76 120.65) (width 0.5) (layer B.Cu) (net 11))
 (segment (start 149.098 123.19) (end 146.558 120.65) (width 0.5) (layer B.Cu) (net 11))
 (segment (start 152.654 125.222) (end 150.622 123.19) (width 0.5) (layer B.Cu) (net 11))
 (segment (start 150.622 123.19) (end 149.098 123.19) (width 0.5) (layer B.Cu) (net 11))
 (segment (start 158.408001 124.372001) (end 157.138001 124.372001) (width 0.5) (layer B.Cu) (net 12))
 (segment (start 159.258 125.222) (end 158.408001 124.372001) (width 0.5) (layer B.Cu) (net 12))
 (segment (start 157.138001 124.372001) (end 156.21 123.444) (width 0.5) (layer B.Cu) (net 12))
 (segment (start 156.21 123.444) (end 156.21 122.682) (width 0.5) (layer B.Cu) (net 12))
 (segment (start 156.21 122.682) (end 155.448 121.92) (width 0.5) (layer B.Cu) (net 12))
 (segment (start 155.448 121.92) (end 149.606 121.92) (width 0.5) (layer B.Cu) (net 12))
 (segment (start 149.606 121.92) (end 147.066 119.38) (width 0.5) (layer B.Cu) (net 12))
 (segment (start 147.066 119.38) (end 114.808 119.38) (width 0.5) (layer B.Cu) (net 12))
 (segment (start 113.792 118.364) (end 113.792 116.586) (width 0.5) (layer B.Cu) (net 12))
 (segment (start 114.808 119.38) (end 113.792 118.364) (width 0.5) (layer B.Cu) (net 12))
 (segment (start 106.172 127.254) (end 106.172 116.586) (width 1) (layer B.Cu) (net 9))
 (segment (start 111.506 132.588) (end 106.172 127.254) (width 1) (layer B.Cu) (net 9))
 (segment (start 134.941919 132.588) (end 111.506 132.588) (width 1) (layer B.Cu) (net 9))
 (segment (start 136.398 132.842) (end 135.195919 132.842) (width 1) (layer B.Cu) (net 9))
 (segment (start 135.195919 132.842) (end 134.941919 132.588) (width 1) (layer B.Cu) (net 9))
 (segment (start 144.78 132.842) (end 136.398 132.842) (width 1) (layer B.Cu) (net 9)))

